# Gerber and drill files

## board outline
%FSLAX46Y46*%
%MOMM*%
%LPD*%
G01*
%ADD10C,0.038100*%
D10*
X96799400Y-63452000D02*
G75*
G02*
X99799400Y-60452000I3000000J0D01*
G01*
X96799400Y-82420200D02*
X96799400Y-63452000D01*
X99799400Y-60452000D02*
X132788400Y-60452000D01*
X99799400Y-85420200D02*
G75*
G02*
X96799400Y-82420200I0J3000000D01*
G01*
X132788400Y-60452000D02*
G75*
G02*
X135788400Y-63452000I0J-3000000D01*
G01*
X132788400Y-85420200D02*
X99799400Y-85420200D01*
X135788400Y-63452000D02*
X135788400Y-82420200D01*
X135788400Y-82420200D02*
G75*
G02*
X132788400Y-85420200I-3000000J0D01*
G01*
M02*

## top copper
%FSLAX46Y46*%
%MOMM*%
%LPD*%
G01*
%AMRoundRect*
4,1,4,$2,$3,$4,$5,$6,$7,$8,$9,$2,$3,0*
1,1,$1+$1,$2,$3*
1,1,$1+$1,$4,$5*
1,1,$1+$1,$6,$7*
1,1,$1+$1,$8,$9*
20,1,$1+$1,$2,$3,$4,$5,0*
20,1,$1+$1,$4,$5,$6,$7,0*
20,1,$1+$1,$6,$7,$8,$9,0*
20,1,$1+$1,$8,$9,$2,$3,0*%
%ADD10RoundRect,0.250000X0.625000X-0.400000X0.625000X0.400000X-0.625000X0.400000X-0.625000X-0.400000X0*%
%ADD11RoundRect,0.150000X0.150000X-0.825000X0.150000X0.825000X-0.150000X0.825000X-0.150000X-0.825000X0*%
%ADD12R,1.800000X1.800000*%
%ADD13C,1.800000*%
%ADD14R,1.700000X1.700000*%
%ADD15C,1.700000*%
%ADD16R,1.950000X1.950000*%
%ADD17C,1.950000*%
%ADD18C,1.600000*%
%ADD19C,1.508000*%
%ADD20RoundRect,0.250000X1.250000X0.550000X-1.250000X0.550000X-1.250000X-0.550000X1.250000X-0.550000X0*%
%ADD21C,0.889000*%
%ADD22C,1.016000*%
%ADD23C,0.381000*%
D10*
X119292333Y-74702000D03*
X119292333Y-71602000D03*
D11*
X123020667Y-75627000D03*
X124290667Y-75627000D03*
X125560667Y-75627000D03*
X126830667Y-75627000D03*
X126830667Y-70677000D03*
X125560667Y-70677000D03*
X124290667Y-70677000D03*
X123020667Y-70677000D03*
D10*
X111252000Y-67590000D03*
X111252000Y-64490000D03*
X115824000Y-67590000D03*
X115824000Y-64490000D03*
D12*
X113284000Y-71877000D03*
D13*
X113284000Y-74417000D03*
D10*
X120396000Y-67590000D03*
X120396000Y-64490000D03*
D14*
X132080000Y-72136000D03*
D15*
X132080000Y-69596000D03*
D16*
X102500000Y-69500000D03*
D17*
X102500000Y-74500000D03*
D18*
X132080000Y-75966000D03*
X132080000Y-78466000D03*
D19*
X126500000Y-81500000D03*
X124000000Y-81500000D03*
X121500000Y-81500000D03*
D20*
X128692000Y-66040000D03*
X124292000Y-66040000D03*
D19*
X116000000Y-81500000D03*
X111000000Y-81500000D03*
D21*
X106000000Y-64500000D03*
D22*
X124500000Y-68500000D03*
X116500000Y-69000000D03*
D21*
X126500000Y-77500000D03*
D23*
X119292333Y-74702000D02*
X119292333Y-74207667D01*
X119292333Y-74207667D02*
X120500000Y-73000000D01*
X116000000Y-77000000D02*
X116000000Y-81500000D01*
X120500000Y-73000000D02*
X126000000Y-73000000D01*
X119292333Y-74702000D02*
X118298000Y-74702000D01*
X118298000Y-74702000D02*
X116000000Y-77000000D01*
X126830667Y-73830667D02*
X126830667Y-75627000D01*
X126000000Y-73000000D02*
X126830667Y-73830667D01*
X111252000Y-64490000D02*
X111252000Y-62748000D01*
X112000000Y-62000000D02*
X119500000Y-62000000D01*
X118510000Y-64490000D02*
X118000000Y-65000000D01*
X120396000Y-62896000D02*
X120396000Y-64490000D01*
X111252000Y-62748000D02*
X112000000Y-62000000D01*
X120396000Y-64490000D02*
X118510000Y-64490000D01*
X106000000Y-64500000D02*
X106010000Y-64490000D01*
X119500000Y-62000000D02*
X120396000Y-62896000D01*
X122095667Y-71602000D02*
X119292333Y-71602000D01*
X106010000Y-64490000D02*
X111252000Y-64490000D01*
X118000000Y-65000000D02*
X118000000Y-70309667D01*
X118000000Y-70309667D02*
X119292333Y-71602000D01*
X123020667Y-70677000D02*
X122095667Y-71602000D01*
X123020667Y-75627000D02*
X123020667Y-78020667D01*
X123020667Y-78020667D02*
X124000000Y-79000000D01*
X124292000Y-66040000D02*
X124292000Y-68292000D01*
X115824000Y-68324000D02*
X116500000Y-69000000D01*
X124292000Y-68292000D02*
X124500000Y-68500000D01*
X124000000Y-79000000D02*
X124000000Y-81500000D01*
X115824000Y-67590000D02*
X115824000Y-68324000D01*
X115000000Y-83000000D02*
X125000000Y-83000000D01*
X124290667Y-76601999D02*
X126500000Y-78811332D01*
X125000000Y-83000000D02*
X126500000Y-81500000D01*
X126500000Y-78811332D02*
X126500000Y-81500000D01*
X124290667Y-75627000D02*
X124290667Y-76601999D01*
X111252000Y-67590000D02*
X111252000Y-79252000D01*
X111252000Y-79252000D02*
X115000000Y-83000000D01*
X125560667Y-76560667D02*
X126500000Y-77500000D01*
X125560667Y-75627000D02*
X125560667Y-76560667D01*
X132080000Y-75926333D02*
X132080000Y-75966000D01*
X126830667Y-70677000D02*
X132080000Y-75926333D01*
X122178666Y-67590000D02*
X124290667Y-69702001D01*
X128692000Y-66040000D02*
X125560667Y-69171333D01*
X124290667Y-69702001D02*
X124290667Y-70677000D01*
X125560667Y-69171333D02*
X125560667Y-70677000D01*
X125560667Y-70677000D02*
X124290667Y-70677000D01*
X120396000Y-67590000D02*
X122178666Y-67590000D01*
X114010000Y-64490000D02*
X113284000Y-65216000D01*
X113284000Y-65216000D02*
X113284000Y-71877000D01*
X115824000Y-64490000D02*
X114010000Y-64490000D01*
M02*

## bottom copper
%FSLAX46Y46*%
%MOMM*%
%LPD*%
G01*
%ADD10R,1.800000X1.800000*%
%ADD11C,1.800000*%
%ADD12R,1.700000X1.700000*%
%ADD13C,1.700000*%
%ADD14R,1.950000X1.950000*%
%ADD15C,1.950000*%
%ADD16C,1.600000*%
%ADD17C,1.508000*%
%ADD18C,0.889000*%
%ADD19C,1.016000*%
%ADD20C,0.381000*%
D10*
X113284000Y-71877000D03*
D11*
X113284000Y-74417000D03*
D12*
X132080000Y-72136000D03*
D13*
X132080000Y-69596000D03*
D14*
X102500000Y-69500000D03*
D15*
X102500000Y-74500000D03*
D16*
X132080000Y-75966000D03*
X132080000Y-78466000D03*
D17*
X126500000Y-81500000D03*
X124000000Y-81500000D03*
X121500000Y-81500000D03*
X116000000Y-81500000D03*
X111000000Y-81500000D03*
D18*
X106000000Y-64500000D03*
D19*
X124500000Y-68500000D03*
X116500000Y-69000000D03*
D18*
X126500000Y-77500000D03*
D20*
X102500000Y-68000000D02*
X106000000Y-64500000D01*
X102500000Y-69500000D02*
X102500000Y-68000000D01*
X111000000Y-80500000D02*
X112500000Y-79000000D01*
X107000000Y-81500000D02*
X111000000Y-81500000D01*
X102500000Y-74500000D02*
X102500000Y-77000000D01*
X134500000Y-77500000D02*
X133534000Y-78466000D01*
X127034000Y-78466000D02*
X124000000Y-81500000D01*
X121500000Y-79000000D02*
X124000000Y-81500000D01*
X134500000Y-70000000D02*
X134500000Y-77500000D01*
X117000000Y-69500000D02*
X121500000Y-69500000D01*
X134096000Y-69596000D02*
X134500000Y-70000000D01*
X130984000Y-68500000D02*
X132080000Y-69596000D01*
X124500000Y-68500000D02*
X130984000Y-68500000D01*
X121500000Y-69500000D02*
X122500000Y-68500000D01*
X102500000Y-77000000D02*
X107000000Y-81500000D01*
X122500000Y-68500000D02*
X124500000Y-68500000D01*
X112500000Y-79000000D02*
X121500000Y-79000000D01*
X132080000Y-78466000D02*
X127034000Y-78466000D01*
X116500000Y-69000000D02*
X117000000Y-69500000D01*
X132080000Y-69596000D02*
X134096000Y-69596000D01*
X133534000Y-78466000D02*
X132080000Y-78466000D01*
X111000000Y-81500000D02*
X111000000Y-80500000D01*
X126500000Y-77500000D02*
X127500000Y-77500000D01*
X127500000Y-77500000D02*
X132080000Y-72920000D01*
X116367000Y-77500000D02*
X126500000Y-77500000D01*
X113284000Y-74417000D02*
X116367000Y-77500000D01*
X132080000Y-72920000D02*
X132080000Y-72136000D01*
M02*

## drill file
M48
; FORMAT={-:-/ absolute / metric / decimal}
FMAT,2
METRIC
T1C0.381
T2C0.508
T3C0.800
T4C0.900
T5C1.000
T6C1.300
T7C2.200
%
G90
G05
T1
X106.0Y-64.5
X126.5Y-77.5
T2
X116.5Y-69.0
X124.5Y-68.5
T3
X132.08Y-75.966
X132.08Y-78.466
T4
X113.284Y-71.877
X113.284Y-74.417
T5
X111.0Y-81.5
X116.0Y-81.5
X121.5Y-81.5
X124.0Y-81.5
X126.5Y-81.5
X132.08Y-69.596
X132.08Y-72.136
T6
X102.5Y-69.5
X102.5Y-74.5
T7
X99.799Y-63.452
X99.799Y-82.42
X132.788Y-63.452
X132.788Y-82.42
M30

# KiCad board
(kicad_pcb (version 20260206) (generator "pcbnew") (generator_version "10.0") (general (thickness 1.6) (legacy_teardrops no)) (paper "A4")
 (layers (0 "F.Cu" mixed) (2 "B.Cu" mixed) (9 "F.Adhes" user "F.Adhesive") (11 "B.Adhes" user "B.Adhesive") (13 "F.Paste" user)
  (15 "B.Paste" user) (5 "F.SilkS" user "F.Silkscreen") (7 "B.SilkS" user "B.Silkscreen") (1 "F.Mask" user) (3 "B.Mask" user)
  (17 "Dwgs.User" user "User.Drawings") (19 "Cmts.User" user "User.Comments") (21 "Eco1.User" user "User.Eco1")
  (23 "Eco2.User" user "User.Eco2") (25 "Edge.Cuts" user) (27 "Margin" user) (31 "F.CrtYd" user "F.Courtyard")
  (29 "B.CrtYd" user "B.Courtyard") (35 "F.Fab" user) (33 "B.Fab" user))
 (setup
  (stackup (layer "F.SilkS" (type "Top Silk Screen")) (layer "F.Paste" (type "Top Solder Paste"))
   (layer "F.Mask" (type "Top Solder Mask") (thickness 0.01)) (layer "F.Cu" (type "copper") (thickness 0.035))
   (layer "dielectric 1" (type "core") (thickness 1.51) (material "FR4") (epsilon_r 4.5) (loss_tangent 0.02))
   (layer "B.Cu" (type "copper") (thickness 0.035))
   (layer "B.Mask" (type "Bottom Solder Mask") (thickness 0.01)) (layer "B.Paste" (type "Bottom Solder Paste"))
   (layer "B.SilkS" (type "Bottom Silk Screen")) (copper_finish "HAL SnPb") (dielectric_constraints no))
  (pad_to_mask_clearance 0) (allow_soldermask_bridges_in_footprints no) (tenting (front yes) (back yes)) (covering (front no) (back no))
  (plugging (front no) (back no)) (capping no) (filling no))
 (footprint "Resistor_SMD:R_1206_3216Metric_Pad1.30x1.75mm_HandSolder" (layer "F.Cu") (at 119.292333 73.152 90)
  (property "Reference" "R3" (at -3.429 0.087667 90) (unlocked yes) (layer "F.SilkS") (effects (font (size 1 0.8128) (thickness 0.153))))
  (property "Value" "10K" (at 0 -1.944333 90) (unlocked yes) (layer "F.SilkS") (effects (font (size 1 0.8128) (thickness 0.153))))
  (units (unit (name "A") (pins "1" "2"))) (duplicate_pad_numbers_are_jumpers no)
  (pad "1" smd roundrect (at -1.55 0 90) (size 1.3 1.75) (layers "F.Cu" "F.Mask" "F.Paste") (roundrect_rratio 0.192308) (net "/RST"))
  (pad "2" smd roundrect (at 1.55 0 90) (size 1.3 1.75) (layers "F.Cu" "F.Mask" "F.Paste") (roundrect_rratio 0.192308) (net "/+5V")))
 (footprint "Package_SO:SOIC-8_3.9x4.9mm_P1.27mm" (layer "F.Cu") (at 124.925667 73.152 90)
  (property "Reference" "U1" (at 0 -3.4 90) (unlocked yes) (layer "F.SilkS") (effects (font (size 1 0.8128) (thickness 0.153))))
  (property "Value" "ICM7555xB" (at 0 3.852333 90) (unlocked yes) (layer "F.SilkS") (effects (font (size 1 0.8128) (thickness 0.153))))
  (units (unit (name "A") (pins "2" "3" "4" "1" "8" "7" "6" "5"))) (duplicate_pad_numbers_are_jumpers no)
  (pad "1" smd roundrect (at -2.475 -1.905 90) (size 1.95 0.6) (layers "F.Cu" "F.Mask" "F.Paste") (roundrect_rratio 0.25) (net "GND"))
  (pad "2" smd roundrect (at -2.475 -0.635 90) (size 1.95 0.6) (layers "F.Cu" "F.Mask" "F.Paste") (roundrect_rratio 0.25) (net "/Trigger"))
  (pad "3" smd roundrect (at -2.475 0.635 90) (size 1.95 0.6) (layers "F.Cu" "F.Mask" "F.Paste") (roundrect_rratio 0.25) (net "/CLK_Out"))
  (pad "4" smd roundrect (at -2.475 1.905 90) (size 1.95 0.6) (layers "F.Cu" "F.Mask" "F.Paste") (roundrect_rratio 0.25) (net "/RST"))
  (pad "5" smd roundrect (at 2.475 1.905 90) (size 1.95 0.6) (layers "F.Cu" "F.Mask" "F.Paste") (roundrect_rratio 0.25)
   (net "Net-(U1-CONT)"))
  (pad "6" smd roundrect (at 2.475 0.635 90) (size 1.95 0.6) (layers "F.Cu" "F.Mask" "F.Paste") (roundrect_rratio 0.25)
   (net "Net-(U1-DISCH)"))
  (pad "7" smd roundrect (at 2.475 -0.635 90) (size 1.95 0.6) (layers "F.Cu" "F.Mask" "F.Paste") (roundrect_rratio 0.25)
   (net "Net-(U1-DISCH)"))
  (pad "8" smd roundrect (at 2.475 -1.905 90) (size 1.95 0.6) (layers "F.Cu" "F.Mask" "F.Paste") (roundrect_rratio 0.25) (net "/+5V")))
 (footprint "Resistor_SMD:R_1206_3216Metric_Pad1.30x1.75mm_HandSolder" (layer "F.Cu") (at 111.252 66.04 90)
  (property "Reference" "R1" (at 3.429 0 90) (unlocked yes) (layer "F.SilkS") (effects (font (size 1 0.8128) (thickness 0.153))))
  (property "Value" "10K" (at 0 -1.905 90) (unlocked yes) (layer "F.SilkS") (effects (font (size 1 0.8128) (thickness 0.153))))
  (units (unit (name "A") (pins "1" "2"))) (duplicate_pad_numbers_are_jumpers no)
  (pad "1" smd roundrect (at -1.55 0 90) (size 1.3 1.75) (layers "F.Cu" "F.Mask" "F.Paste") (roundrect_rratio 0.192308) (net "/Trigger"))
  (pad "2" smd roundrect (at 1.55 0 90) (size 1.3 1.75) (layers "F.Cu" "F.Mask" "F.Paste") (roundrect_rratio 0.192308) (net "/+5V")))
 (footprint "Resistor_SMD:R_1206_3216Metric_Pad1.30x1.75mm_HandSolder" (layer "F.Cu") (at 115.824 66.04 90)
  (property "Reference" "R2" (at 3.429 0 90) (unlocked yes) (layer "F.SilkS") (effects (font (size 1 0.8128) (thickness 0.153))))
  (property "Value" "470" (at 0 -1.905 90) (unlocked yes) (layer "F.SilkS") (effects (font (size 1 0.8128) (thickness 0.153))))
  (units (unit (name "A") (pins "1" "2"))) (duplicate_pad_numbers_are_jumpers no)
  (pad "1" smd roundrect (at -1.55 0 90) (size 1.3 1.75) (layers "F.Cu" "F.Mask" "F.Paste") (roundrect_rratio 0.192308) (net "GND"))
  (pad "2" smd roundrect (at 1.55 0 90) (size 1.3 1.75) (layers "F.Cu" "F.Mask" "F.Paste") (roundrect_rratio 0.192308) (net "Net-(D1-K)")))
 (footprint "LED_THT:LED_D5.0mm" (layer "F.Cu") (at 113.284 71.877 -90)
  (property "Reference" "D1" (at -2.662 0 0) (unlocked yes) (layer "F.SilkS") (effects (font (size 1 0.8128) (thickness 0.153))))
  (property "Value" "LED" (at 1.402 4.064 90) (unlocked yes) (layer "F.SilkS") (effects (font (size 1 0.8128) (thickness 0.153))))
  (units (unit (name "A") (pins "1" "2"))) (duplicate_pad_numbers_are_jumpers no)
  (pad "1" thru_hole rect (at 0 0 270) (size 1.8 1.8) (drill 0.9) (layers "*.Cu" "*.Mask") (remove_unused_layers no) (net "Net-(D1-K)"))
  (pad "2" thru_hole circle (at 2.54 0 270) (size 1.8 1.8) (drill 0.9) (layers "*.Cu" "*.Mask") (remove_unused_layers no) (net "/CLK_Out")))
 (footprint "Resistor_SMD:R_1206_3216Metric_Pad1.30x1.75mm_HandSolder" (layer "F.Cu") (at 120.396 66.04 90)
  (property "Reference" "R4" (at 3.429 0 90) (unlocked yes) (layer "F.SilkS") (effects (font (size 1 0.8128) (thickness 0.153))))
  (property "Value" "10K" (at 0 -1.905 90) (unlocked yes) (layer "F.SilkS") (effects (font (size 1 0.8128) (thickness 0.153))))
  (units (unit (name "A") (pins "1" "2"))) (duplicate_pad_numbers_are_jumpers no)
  (pad "1" smd roundrect (at -1.55 0 90) (size 1.3 1.75) (layers "F.Cu" "F.Mask" "F.Paste") (roundrect_rratio 0.192308)
   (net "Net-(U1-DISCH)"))
  (pad "2" smd roundrect (at 1.55 0 90) (size 1.3 1.75) (layers "F.Cu" "F.Mask" "F.Paste") (roundrect_rratio 0.192308) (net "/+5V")))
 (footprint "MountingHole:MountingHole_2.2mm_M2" (layer "F.Cu") (at 99.7994 63.452)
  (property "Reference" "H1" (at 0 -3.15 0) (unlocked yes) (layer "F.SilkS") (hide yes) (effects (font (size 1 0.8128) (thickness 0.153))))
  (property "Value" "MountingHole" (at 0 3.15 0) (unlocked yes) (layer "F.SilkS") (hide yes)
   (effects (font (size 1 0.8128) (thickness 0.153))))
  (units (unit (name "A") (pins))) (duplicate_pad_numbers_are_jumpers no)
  (pad "" np_thru_hole circle (at 0 0) (size 2.2 2.2) (drill 2.2) (layers "*.Cu" "*.Mask")))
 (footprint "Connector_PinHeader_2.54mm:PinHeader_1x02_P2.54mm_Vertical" (layer "F.Cu") (at 132.08 72.136 180)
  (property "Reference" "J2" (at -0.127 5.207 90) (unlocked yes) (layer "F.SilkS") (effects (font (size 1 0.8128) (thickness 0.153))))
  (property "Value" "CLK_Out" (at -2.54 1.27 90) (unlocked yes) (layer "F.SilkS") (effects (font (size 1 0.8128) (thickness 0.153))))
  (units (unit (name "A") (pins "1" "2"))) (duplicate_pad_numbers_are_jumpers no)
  (pad "1" thru_hole rect (at 0 0 180) (size 1.7 1.7) (drill 1) (layers "*.Cu" "*.Mask") (remove_unused_layers no) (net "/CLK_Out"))
  (pad "2" thru_hole circle (at 0 2.54 180) (size 1.7 1.7) (drill 1) (layers "*.Cu" "*.Mask") (remove_unused_layers no) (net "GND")))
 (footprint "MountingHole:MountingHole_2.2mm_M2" (layer "F.Cu") (at 132.7884 82.4202)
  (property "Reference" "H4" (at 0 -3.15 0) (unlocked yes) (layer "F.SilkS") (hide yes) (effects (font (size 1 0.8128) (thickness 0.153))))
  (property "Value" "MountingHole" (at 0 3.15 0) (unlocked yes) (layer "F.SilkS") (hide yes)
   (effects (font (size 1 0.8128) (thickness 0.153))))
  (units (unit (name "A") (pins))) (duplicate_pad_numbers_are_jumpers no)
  (pad "" np_thru_hole circle (at 0 0) (size 2.2 2.2) (drill 2.2) (layers "*.Cu" "*.Mask")))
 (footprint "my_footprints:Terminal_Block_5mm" (layer "F.Cu") (at 102.5 72 -90)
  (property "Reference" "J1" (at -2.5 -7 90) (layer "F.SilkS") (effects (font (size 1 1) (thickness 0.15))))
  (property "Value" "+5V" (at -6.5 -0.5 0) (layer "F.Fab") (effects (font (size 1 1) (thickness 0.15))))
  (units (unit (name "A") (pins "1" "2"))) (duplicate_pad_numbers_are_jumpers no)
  (pad "1" thru_hole rect (at -2.5 0 270) (size 1.95 1.95) (drill 1.3) (layers "*.Cu" "*.Mask") (remove_unused_layers no) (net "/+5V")
   (solder_mask_margin 0.102))
  (pad "2" thru_hole circle (at 2.5 0 270) (size 1.95 1.95) (drill 1.3) (layers "*.Cu" "*.Mask") (remove_unused_layers no) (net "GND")
   (solder_mask_margin 0.102)))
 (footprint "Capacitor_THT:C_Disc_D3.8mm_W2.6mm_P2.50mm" (layer "F.Cu") (at 132.08 75.966 -90)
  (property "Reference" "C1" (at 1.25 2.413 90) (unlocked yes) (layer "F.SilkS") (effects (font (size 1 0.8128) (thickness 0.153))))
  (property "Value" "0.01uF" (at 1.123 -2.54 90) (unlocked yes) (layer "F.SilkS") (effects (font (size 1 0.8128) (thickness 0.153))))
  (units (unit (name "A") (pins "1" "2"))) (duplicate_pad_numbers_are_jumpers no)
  (pad "1" thru_hole circle (at 0 0 270) (size 1.6 1.6) (drill 0.8) (layers "*.Cu" "*.Mask") (remove_unused_layers no) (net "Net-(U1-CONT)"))
  (pad "2" thru_hole circle (at 2.5 0 270) (size 1.6 1.6) (drill 0.8) (layers "*.Cu" "*.Mask") (remove_unused_layers no) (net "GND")))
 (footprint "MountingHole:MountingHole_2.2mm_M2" (layer "F.Cu") (at 132.7884 63.452)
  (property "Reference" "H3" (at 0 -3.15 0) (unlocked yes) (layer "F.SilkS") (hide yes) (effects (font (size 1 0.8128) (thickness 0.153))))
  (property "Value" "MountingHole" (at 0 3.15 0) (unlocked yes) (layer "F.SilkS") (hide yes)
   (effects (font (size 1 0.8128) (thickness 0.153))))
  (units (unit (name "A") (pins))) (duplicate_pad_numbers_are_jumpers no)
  (pad "" np_thru_hole circle (at 0 0) (size 2.2 2.2) (drill 2.2) (layers "*.Cu" "*.Mask")))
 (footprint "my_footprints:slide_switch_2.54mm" (layer "F.Cu") (at 124 81.5 180)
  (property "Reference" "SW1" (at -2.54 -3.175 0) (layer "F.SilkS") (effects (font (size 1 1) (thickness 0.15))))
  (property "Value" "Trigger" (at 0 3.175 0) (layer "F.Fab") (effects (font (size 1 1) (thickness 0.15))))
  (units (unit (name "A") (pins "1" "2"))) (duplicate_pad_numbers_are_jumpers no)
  (pad "1" thru_hole circle (at -2.5 0 180) (size 1.508 1.508) (drill 1) (layers "*.Cu" "*.Mask") (remove_unused_layers no) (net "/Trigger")
   (solder_mask_margin 0.102))
  (pad "2" thru_hole circle (at 0 0 180) (size 1.508 1.508) (drill 1) (layers "*.Cu" "*.Mask") (remove_unused_layers no) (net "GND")
   (solder_mask_margin 0.102))
  (pad "3" thru_hole circle (at 2.5 0 180) (size 1.508 1.508) (drill 1) (layers "*.Cu" "*.Mask") (remove_unused_layers no)
   (solder_mask_margin 0.102)))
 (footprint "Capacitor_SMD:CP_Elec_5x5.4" (layer "F.Cu") (at 126.492 66.04 180)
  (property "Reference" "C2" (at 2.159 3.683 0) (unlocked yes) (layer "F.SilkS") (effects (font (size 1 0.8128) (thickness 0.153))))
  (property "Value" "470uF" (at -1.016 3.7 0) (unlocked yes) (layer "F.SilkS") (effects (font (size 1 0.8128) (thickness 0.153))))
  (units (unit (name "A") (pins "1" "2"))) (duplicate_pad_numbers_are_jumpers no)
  (pad "1" smd roundrect (at -2.2 0 180) (size 3 1.6) (layers "F.Cu" "F.Mask" "F.Paste") (roundrect_rratio 0.15625) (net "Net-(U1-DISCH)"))
  (pad "2" smd roundrect (at 2.2 0 180) (size 3 1.6) (layers "F.Cu" "F.Mask" "F.Paste") (roundrect_rratio 0.15625) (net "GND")))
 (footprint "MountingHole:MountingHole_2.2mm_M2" (layer "F.Cu") (at 99.7994 82.4202)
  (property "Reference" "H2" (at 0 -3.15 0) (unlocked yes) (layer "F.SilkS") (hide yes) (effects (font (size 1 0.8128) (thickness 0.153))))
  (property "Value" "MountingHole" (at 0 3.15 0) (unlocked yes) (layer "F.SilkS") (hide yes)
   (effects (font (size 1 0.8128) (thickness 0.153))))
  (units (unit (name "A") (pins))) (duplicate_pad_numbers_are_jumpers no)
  (pad "" np_thru_hole circle (at 0 0) (size 2.2 2.2) (drill 2.2) (layers "*.Cu" "*.Mask")))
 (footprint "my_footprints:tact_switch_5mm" (layer "F.Cu") (at 113.5 81.5 180)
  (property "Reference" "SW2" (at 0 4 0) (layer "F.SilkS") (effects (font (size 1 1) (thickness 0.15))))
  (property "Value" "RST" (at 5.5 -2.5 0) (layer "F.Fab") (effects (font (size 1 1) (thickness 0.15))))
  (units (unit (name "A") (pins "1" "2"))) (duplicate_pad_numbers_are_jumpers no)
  (pad "1" thru_hole circle (at -2.5 0 180) (size 1.508 1.508) (drill 1) (layers "*.Cu" "*.Mask") (remove_unused_layers no) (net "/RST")
   (solder_mask_margin 0.102))
  (pad "2" thru_hole circle (at 2.5 0 180) (size 1.508 1.508) (drill 1) (layers "*.Cu" "*.Mask") (remove_unused_layers no) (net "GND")
   (solder_mask_margin 0.102)))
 (gr_arc (start 96.7994 63.452) (mid 97.67808 61.33068) (end 99.7994 60.452) (stroke (width 0.0381) (type default)) (layer "Edge.Cuts"))
 (gr_line (start 96.7994 82.4202) (end 96.7994 63.452) (stroke (width 0.0381) (type default)) (layer "Edge.Cuts"))
 (gr_line (start 99.7994 60.452) (end 132.7884 60.452) (stroke (width 0.0381) (type default)) (layer "Edge.Cuts"))
 (gr_arc (start 99.7994 85.4202) (mid 97.67808 84.54152) (end 96.7994 82.4202) (stroke (width 0.0381) (type default)) (layer "Edge.Cuts"))
 (gr_arc (start 132.7884 60.452) (mid 134.90972 61.33068) (end 135.7884 63.452) (stroke (width 0.0381) (type default)) (layer "Edge.Cuts"))
 (gr_line (start 132.7884 85.4202) (end 99.7994 85.4202) (stroke (width 0.0381) (type default)) (layer "Edge.Cuts"))
 (gr_line (start 135.7884 63.452) (end 135.7884 82.4202) (stroke (width 0.0381) (type default)) (layer "Edge.Cuts"))
 (gr_arc (start 135.7884 82.4202) (mid 134.90972 84.54152) (end 132.7884 85.4202) (stroke (width 0.0381) (type default)) (layer "Edge.Cuts"))
 (segment (start 119.292333 74.702) (end 119.292333 74.207667) (width 0.381) (layer "F.Cu") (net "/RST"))
 (segment (start 119.292333 74.207667) (end 120.5 73) (width 0.381) (layer "F.Cu") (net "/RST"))
 (segment (start 116 77) (end 116 81.5) (width 0.381) (layer "F.Cu") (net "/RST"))
 (segment (start 120.5 73) (end 126 73) (width 0.381) (layer "F.Cu") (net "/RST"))
 (segment (start 119.292333 74.702) (end 118.298 74.702) (width 0.381) (layer "F.Cu") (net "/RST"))
 (segment (start 118.298 74.702) (end 116 77) (width 0.381) (layer "F.Cu") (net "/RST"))
 (segment (start 126.830667 73.830667) (end 126.830667 75.627) (width 0.381) (layer "F.Cu") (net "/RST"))
 (segment (start 126 73) (end 126.830667 73.830667) (width 0.381) (layer "F.Cu") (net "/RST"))
 (segment (start 111.252 64.49) (end 111.252 62.748) (width 0.381) (layer "F.Cu") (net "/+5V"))
 (segment (start 112 62) (end 119.5 62) (width 0.381) (layer "F.Cu") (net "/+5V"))
 (segment (start 118.51 64.49) (end 118 65) (width 0.381) (layer "F.Cu") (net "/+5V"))
 (segment (start 120.396 62.896) (end 120.396 64.49) (width 0.381) (layer "F.Cu") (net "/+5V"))
 (segment (start 111.252 62.748) (end 112 62) (width 0.381) (layer "F.Cu") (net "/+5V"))
 (segment (start 120.396 64.49) (end 118.51 64.49) (width 0.381) (layer "F.Cu") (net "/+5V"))
 (segment (start 106 64.5) (end 106.01 64.49) (width 0.381) (layer "F.Cu") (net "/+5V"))
 (segment (start 119.5 62) (end 120.396 62.896) (width 0.381) (layer "F.Cu") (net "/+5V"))
 (segment (start 122.095667 71.602) (end 119.292333 71.602) (width 0.381) (layer "F.Cu") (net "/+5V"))
 (segment (start 106.01 64.49) (end 111.252 64.49) (width 0.381) (layer "F.Cu") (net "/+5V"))
 (segment (start 118 65) (end 118 70.309667) (width 0.381) (layer "F.Cu") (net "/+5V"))
 (segment (start 118 70.309667) (end 119.292333 71.602) (width 0.381) (layer "F.Cu") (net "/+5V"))
 (segment (start 123.020667 70.677) (end 122.095667 71.602) (width 0.381) (layer "F.Cu") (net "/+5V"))
 (via (at 106 64.5) (size 0.889) (drill 0.381) (layers "F.Cu" "B.Cu") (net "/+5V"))
 (segment (start 102.5 68) (end 106 64.5) (width 0.381) (layer "B.Cu") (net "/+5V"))
 (segment (start 102.5 69.5) (end 102.5 68) (width 0.381) (layer "B.Cu") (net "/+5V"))
 (segment (start 123.020667 75.627) (end 123.020667 78.020667) (width 0.381) (layer "F.Cu") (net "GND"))
 (segment (start 123.020667 78.020667) (end 124 79) (width 0.381) (layer "F.Cu") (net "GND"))
 (segment (start 124.292 66.04) (end 124.292 68.292) (width 0.381) (layer "F.Cu") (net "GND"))
 (segment (start 115.824 68.324) (end 116.5 69) (width 0.381) (layer "F.Cu") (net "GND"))
 (segment (start 124.292 68.292) (end 124.5 68.5) (width 0.381) (layer "F.Cu") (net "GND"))
 (segment (start 124 79) (end 124 81.5) (width 0.381) (layer "F.Cu") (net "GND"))
 (segment (start 115.824 67.59) (end 115.824 68.324) (width 0.381) (layer "F.Cu") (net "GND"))
 (via (at 124.5 68.5) (size 1.016) (drill 0.508) (layers "F.Cu" "B.Cu") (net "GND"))
 (via (at 116.5 69) (size 1.016) (drill 0.508) (layers "F.Cu" "B.Cu") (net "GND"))
 (segment (start 111 80.5) (end 112.5 79) (width 0.381) (layer "B.Cu") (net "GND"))
 (segment (start 107 81.5) (end 111 81.5) (width 0.381) (layer "B.Cu") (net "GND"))
 (segment (start 102.5 74.5) (end 102.5 77) (width 0.381) (layer "B.Cu") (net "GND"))
 (segment (start 134.5 77.5) (end 133.534 78.466) (width 0.381) (layer "B.Cu") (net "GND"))
 (segment (start 127.034 78.466) (end 124 81.5) (width 0.381) (layer "B.Cu") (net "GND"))
 (segment (start 121.5 79) (end 124 81.5) (width 0.381) (layer "B.Cu") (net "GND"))
 (segment (start 134.5 70) (end 134.5 77.5) (width 0.381) (layer "B.Cu") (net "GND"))
 (segment (start 117 69.5) (end 121.5 69.5) (width 0.381) (layer "B.Cu") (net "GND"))
 (segment (start 134.096 69.596) (end 134.5 70) (width 0.381) (layer "B.Cu") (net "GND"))
 (segment (start 130.984 68.5) (end 132.08 69.596) (width 0.381) (layer "B.Cu") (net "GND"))
 (segment (start 124.5 68.5) (end 130.984 68.5) (width 0.381) (layer "B.Cu") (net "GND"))
 (segment (start 121.5 69.5) (end 122.5 68.5) (width 0.381) (layer "B.Cu") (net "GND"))
 (segment (start 102.5 77) (end 107 81.5) (width 0.381) (layer "B.Cu") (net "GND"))
 (segment (start 122.5 68.5) (end 124.5 68.5) (width 0.381) (layer "B.Cu") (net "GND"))
 (segment (start 112.5 79) (end 121.5 79) (width 0.381) (layer "B.Cu") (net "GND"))
 (segment (start 132.08 78.466) (end 127.034 78.466) (width 0.381) (layer "B.Cu") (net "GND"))
 (segment (start 116.5 69) (end 117 69.5) (width 0.381) (layer "B.Cu") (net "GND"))
 (segment (start 132.08 69.596) (end 134.096 69.596) (width 0.381) (layer "B.Cu") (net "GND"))
 (segment (start 133.534 78.466) (end 132.08 78.466) (width 0.381) (layer "B.Cu") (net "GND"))
 (segment (start 111 81.5) (end 111 80.5) (width 0.381) (layer "B.Cu") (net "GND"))
 (segment (start 115 83) (end 125 83) (width 0.381) (layer "F.Cu") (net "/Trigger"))
 (segment (start 124.290667 76.601999) (end 126.5 78.811332) (width 0.381) (layer "F.Cu") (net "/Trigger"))
 (segment (start 125 83) (end 126.5 81.5) (width 0.381) (layer "F.Cu") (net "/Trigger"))
 (segment (start 126.5 78.811332) (end 126.5 81.5) (width 0.381) (layer "F.Cu") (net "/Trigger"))
 (segment (start 124.290667 75.627) (end 124.290667 76.601999) (width 0.381) (layer "F.Cu") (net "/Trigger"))
 (segment (start 111.252 67.59) (end 111.252 79.252) (width 0.381) (layer "F.Cu") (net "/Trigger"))
 (segment (start 111.252 79.252) (end 115 83) (width 0.381) (layer "F.Cu") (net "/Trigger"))
 (segment (start 125.560667 76.560667) (end 126.5 77.5) (width 0.381) (layer "F.Cu") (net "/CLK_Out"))
 (segment (start 125.560667 75.627) (end 125.560667 76.560667) (width 0.381) (layer "F.Cu") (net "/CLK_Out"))
 (via (at 126.5 77.5) (size 0.889) (drill 0.381) (layers "F.Cu" "B.Cu") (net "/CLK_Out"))
 (segment (start 126.5 77.5) (end 127.5 77.5) (width 0.381) (layer "B.Cu") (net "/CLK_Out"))
 (segment (start 127.5 77.5) (end 132.08 72.92) (width 0.381) (layer "B.Cu") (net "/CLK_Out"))
 (segment (start 116.367 77.5) (end 126.5 77.5) (width 0.381) (layer "B.Cu") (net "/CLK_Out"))
 (segment (start 113.284 74.417) (end 116.367 77.5) (width 0.381) (layer "B.Cu") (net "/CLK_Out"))
 (segment (start 132.08 72.92) (end 132.08 72.136) (width 0.381) (layer "B.Cu") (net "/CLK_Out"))
 (segment (start 132.08 75.926333) (end 132.08 75.966) (width 0.381) (layer "F.Cu") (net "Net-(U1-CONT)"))
 (segment (start 126.830667 70.677) (end 132.08 75.926333) (width 0.381) (layer "F.Cu") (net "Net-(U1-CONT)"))
 (segment (start 122.178666 67.59) (end 124.290667 69.702001) (width 0.381) (layer "F.Cu") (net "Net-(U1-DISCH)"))
 (segment (start 128.692 66.04) (end 125.560667 69.171333) (width 0.381) (layer "F.Cu") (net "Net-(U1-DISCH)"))
 (segment (start 124.290667 69.702001) (end 124.290667 70.677) (width 0.381) (layer "F.Cu") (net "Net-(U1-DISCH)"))
 (segment (start 125.560667 69.171333) (end 125.560667 70.677) (width 0.381) (layer "F.Cu") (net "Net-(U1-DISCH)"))
 (segment (start 125.560667 70.677) (end 124.290667 70.677) (width 0.381) (layer "F.Cu") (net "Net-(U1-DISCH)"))
 (segment (start 120.396 67.59) (end 122.178666 67.59) (width 0.381) (layer "F.Cu") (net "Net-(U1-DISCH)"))
 (segment (start 114.01 64.49) (end 113.284 65.216) (width 0.381) (layer "F.Cu") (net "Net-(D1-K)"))
 (segment (start 113.284 65.216) (end 113.284 71.877) (width 0.381) (layer "F.Cu") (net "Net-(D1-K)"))
 (segment (start 115.824 64.49) (end 114.01 64.49) (width 0.381) (layer "F.Cu") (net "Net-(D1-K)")))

